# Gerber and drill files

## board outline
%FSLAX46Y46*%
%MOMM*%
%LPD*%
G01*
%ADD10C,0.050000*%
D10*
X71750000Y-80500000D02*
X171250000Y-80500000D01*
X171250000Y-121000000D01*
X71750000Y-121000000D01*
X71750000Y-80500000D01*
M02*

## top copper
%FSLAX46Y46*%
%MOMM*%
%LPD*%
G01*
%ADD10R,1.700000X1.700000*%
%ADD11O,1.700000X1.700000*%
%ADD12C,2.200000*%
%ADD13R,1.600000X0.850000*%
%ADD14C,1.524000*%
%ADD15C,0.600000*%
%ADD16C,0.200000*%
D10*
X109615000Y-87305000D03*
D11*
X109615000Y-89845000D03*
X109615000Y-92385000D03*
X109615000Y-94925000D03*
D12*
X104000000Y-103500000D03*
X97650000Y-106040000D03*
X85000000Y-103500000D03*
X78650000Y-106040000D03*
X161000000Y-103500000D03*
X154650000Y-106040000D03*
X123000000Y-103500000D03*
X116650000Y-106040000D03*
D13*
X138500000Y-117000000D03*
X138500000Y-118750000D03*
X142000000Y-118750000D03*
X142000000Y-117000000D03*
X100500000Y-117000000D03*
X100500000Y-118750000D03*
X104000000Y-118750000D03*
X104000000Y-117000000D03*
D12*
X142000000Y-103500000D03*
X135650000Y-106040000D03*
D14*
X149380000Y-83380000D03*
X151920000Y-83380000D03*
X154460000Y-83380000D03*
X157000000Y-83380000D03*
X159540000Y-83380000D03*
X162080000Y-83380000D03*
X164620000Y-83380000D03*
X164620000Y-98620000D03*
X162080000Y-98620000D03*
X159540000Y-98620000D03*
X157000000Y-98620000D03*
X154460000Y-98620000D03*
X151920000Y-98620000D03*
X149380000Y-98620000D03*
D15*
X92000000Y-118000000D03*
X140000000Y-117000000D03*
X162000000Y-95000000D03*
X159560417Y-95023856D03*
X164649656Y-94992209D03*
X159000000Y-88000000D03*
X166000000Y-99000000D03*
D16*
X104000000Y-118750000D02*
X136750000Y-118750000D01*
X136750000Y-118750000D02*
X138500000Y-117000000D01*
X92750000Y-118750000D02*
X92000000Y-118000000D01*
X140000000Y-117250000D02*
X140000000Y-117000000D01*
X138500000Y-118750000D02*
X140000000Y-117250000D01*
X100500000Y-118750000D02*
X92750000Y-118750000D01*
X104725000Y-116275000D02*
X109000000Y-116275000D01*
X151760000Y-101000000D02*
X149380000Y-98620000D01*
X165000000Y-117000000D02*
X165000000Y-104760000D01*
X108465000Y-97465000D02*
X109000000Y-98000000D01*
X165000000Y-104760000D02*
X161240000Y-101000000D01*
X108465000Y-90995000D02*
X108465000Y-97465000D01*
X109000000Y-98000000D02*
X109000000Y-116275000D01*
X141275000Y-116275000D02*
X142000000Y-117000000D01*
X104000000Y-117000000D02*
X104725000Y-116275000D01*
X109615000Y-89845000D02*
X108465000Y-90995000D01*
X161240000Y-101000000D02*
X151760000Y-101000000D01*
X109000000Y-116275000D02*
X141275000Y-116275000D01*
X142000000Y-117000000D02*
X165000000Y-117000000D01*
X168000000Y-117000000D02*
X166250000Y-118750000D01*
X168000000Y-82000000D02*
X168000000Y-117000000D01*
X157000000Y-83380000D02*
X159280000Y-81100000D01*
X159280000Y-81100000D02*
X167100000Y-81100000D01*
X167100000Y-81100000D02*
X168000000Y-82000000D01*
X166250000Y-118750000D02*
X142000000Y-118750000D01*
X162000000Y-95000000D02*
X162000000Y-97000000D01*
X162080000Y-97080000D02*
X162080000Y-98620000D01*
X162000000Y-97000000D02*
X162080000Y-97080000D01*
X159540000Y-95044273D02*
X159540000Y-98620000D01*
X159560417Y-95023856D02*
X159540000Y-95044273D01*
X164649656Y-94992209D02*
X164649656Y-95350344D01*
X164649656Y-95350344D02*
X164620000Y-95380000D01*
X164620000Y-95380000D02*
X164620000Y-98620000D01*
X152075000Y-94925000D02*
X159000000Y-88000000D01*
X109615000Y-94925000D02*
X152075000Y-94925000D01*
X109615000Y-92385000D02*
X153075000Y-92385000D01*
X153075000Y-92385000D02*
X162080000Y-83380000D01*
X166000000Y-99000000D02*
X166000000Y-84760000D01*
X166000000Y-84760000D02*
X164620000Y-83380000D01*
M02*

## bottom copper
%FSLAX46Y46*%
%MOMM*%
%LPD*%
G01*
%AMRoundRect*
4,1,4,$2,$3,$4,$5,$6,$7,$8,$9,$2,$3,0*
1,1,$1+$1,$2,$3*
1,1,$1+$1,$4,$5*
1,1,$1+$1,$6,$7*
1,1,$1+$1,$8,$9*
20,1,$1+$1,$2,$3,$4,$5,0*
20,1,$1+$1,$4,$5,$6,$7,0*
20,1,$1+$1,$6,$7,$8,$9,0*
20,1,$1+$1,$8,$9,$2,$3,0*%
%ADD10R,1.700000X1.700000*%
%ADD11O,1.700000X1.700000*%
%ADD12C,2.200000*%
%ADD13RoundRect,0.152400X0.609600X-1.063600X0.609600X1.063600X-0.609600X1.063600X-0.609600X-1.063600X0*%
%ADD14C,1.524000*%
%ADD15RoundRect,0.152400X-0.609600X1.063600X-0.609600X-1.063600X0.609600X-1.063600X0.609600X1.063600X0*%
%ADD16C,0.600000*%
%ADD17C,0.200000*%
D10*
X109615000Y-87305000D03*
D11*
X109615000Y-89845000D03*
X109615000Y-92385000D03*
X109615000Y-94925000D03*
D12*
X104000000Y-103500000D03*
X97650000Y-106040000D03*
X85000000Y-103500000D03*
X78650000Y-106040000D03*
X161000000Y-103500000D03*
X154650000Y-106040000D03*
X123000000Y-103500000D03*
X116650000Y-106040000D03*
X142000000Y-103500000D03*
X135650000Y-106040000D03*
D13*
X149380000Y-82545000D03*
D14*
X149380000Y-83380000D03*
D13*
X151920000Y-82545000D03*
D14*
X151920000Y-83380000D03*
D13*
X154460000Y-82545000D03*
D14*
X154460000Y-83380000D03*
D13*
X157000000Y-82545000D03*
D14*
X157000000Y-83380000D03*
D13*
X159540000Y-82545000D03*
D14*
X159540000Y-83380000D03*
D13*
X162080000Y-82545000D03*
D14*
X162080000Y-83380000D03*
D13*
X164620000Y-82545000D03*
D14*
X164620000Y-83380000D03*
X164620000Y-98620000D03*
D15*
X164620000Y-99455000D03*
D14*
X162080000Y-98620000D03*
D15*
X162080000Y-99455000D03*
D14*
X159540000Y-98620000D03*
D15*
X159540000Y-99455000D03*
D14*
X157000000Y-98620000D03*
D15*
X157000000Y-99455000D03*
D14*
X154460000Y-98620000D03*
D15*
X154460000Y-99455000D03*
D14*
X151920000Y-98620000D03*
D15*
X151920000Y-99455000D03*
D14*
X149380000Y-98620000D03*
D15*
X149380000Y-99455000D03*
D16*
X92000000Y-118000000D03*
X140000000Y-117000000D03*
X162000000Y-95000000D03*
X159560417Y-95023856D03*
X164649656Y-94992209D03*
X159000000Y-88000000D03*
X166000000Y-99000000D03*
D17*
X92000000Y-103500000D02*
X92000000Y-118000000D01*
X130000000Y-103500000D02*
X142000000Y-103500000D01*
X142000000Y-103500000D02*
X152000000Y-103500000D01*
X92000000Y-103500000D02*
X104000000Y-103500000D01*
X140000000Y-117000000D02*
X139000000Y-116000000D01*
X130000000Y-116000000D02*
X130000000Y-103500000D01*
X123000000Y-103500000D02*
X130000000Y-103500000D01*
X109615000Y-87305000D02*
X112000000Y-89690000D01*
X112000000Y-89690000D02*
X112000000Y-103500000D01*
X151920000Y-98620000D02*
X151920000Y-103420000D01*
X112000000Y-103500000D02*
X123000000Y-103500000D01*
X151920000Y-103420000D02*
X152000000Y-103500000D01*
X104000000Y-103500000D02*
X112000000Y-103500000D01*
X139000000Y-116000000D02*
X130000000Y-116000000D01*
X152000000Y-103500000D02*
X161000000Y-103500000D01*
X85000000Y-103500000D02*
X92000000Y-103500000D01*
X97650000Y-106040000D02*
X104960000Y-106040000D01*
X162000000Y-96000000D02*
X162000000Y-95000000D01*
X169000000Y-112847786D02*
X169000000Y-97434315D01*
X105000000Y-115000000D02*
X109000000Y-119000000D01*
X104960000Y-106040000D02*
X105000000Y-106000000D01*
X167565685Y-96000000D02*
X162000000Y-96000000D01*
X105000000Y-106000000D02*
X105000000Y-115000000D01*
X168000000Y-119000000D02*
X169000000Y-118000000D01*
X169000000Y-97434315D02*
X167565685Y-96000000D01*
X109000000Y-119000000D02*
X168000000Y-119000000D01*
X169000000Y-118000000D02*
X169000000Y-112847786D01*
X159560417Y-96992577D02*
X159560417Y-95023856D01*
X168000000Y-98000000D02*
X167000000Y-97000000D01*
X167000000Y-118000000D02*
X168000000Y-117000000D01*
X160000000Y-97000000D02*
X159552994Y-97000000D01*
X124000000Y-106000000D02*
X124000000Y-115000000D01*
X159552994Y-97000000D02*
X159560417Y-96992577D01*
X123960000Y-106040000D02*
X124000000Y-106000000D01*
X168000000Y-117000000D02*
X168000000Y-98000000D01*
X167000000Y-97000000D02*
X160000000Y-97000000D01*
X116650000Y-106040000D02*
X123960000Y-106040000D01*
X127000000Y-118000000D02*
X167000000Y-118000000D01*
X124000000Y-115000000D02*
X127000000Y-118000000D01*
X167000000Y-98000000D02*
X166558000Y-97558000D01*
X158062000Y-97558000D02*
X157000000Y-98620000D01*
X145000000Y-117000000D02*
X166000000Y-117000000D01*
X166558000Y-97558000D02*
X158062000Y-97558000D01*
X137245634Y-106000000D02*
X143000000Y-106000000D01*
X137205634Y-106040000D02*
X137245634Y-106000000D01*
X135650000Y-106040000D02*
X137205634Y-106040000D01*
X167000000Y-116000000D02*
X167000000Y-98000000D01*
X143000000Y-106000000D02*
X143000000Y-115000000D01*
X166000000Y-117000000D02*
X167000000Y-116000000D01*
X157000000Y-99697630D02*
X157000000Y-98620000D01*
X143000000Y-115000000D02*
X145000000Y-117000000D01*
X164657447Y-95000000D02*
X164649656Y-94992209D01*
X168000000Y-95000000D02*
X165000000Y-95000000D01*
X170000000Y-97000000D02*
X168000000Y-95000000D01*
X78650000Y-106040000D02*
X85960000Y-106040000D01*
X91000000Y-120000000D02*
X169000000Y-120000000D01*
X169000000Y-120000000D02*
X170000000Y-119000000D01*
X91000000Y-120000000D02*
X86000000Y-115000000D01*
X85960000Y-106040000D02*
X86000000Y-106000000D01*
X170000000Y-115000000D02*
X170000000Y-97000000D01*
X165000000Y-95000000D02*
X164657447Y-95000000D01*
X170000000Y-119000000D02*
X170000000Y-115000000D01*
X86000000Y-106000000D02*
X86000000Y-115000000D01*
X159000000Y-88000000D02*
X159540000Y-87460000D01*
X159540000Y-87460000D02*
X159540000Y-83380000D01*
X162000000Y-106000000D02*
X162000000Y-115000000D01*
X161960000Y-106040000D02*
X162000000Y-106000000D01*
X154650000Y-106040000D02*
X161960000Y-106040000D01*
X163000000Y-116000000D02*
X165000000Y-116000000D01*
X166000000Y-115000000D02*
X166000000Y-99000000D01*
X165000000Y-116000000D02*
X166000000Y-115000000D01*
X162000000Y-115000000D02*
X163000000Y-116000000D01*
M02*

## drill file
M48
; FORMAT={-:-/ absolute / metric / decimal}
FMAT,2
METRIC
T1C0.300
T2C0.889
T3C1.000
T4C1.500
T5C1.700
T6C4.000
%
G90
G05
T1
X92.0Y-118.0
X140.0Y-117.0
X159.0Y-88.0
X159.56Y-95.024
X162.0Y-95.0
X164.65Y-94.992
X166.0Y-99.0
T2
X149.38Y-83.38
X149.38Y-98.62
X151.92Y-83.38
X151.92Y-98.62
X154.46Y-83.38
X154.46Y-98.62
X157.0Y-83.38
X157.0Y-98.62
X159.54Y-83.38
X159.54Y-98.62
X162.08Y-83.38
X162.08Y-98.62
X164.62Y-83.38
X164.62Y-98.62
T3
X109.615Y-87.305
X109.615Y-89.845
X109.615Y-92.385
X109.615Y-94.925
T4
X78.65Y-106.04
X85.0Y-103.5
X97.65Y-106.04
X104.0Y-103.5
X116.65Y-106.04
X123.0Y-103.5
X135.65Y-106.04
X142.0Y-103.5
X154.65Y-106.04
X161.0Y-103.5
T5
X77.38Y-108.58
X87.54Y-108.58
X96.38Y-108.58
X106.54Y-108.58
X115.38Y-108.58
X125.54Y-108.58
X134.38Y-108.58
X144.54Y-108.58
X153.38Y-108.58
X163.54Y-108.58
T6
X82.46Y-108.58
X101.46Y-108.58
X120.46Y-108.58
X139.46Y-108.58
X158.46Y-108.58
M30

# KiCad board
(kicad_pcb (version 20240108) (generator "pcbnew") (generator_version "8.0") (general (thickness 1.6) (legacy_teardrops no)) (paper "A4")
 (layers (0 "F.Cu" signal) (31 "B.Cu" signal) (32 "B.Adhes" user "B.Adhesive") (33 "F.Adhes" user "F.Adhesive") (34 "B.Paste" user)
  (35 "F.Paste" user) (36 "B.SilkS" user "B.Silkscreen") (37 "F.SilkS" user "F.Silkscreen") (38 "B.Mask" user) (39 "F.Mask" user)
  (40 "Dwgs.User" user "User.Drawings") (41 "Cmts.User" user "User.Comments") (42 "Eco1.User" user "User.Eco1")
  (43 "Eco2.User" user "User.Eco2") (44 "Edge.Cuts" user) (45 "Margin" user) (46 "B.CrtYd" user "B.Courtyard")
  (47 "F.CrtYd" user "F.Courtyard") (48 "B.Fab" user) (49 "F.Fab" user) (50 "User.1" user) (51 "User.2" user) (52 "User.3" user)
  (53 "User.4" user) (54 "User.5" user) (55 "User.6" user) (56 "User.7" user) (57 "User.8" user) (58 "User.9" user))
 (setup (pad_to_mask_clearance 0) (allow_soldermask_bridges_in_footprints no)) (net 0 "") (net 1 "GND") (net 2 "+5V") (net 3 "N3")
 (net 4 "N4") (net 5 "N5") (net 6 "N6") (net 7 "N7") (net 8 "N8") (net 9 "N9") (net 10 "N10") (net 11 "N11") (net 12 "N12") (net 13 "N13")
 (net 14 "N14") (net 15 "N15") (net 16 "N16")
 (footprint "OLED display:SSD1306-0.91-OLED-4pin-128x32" (layer "F.Cu") (at 73.115 85.115)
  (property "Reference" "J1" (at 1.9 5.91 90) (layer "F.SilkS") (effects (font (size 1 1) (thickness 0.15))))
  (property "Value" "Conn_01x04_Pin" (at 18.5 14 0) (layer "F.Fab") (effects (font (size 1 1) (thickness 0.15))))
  (pad "1" thru_hole rect (at 36.5 2.19) (size 1.7 1.7) (drill 1) (layers "*.Cu" "*.Mask") (remove_unused_layers no) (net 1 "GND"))
  (pad "2" thru_hole oval (at 36.5 4.73) (size 1.7 1.7) (drill 1) (layers "*.Cu" "*.Mask") (remove_unused_layers no) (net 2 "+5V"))
  (pad "3" thru_hole oval (at 36.5 7.27) (size 1.7 1.7) (drill 1) (layers "*.Cu" "*.Mask") (remove_unused_layers no) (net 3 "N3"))
  (pad "4" thru_hole oval (at 36.5 9.81) (size 1.7 1.7) (drill 1) (layers "*.Cu" "*.Mask") (remove_unused_layers no) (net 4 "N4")))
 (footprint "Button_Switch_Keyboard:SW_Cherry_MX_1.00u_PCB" (layer "F.Cu") (at 104 103.5)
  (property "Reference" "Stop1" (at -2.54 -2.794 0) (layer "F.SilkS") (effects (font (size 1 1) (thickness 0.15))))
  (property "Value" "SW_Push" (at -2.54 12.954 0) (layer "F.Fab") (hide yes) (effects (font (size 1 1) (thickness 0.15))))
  (pad "" np_thru_hole circle (at -7.62 5.08) (size 1.7 1.7) (drill 1.7) (layers "*.Cu" "*.Mask"))
  (pad "" np_thru_hole circle (at -2.54 5.08) (size 4 4) (drill 4) (layers "*.Cu" "*.Mask"))
  (pad "" np_thru_hole circle (at 2.54 5.08) (size 1.7 1.7) (drill 1.7) (layers "*.Cu" "*.Mask"))
  (pad "1" thru_hole circle (at 0 0) (size 2.2 2.2) (drill 1.5) (layers "*.Cu" "*.Mask") (remove_unused_layers no) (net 1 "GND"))
  (pad "2" thru_hole circle (at -6.35 2.54) (size 2.2 2.2) (drill 1.5) (layers "*.Cu" "*.Mask") (remove_unused_layers no) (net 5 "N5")))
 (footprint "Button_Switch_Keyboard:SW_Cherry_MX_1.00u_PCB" (layer "F.Cu") (at 85 103.5)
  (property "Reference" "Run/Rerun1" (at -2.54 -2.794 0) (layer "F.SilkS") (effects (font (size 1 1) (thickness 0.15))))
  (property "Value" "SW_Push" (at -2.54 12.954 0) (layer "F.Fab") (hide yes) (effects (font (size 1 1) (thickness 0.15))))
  (pad "" np_thru_hole circle (at -7.62 5.08) (size 1.7 1.7) (drill 1.7) (layers "*.Cu" "*.Mask"))
  (pad "" np_thru_hole circle (at -2.54 5.08) (size 4 4) (drill 4) (layers "*.Cu" "*.Mask"))
  (pad "" np_thru_hole circle (at 2.54 5.08) (size 1.7 1.7) (drill 1.7) (layers "*.Cu" "*.Mask"))
  (pad "1" thru_hole circle (at 0 0) (size 2.2 2.2) (drill 1.5) (layers "*.Cu" "*.Mask") (remove_unused_layers no) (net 1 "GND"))
  (pad "2" thru_hole circle (at -6.35 2.54) (size 2.2 2.2) (drill 1.5) (layers "*.Cu" "*.Mask") (remove_unused_layers no) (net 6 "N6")))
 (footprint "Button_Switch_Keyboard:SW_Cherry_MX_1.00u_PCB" (layer "F.Cu") (at 161 103.5)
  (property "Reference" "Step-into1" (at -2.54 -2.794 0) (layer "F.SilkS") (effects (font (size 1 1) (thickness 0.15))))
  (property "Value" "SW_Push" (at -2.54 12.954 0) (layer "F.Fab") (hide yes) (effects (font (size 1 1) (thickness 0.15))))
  (pad "" np_thru_hole circle (at -7.62 5.08) (size 1.7 1.7) (drill 1.7) (layers "*.Cu" "*.Mask"))
  (pad "" np_thru_hole circle (at -2.54 5.08) (size 4 4) (drill 4) (layers "*.Cu" "*.Mask"))
  (pad "" np_thru_hole circle (at 2.54 5.08) (size 1.7 1.7) (drill 1.7) (layers "*.Cu" "*.Mask"))
  (pad "1" thru_hole circle (at 0 0) (size 2.2 2.2) (drill 1.5) (layers "*.Cu" "*.Mask") (remove_unused_layers no) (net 1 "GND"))
  (pad "2" thru_hole circle (at -6.35 2.54) (size 2.2 2.2) (drill 1.5) (layers "*.Cu" "*.Mask") (remove_unused_layers no) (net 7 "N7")))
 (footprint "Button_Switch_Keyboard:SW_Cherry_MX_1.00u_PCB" (layer "F.Cu") (at 123 103.5)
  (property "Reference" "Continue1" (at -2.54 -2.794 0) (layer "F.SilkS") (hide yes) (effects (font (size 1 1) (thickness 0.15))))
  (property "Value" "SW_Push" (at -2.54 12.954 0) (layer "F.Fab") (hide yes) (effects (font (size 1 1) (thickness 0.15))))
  (pad "" np_thru_hole circle (at -7.62 5.08) (size 1.7 1.7) (drill 1.7) (layers "*.Cu" "*.Mask"))
  (pad "" np_thru_hole circle (at -2.54 5.08) (size 4 4) (drill 4) (layers "*.Cu" "*.Mask"))
  (pad "" np_thru_hole circle (at 2.54 5.08) (size 1.7 1.7) (drill 1.7) (layers "*.Cu" "*.Mask"))
  (pad "1" thru_hole circle (at 0 0) (size 2.2 2.2) (drill 1.5) (layers "*.Cu" "*.Mask") (remove_unused_layers no) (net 1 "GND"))
  (pad "2" thru_hole circle (at -6.35 2.54) (size 2.2 2.2) (drill 1.5) (layers "*.Cu" "*.Mask") (remove_unused_layers no) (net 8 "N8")))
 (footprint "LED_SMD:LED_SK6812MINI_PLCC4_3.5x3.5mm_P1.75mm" (layer "F.Cu") (at 140.25 117.875)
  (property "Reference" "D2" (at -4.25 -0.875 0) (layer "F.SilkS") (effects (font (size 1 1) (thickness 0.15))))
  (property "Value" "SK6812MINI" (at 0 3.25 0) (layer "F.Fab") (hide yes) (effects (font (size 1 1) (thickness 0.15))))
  (pad "1" smd rect (at -1.75 -0.875) (size 1.6 0.85) (layers "F.Cu" "F.Paste" "F.Mask") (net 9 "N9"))
  (pad "2" smd rect (at -1.75 0.875) (size 1.6 0.85) (layers "F.Cu" "F.Paste" "F.Mask") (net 1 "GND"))
  (pad "3" smd rect (at 1.75 0.875) (size 1.6 0.85) (layers "F.Cu" "F.Paste" "F.Mask") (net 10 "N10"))
  (pad "4" smd rect (at 1.75 -0.875) (size 1.6 0.85) (layers "F.Cu" "F.Paste" "F.Mask") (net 2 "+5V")))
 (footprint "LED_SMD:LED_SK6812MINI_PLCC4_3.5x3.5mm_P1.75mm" (layer "F.Cu") (at 102.25 117.875)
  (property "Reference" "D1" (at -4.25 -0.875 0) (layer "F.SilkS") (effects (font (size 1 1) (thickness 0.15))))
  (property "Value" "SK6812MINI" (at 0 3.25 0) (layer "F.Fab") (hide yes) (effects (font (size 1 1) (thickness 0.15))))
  (pad "1" smd rect (at -1.75 -0.875) (size 1.6 0.85) (layers "F.Cu" "F.Paste" "F.Mask") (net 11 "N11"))
  (pad "2" smd rect (at -1.75 0.875) (size 1.6 0.85) (layers "F.Cu" "F.Paste" "F.Mask") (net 1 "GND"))
  (pad "3" smd rect (at 1.75 0.875) (size 1.6 0.85) (layers "F.Cu" "F.Paste" "F.Mask") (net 9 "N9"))
  (pad "4" smd rect (at 1.75 -0.875) (size 1.6 0.85) (layers "F.Cu" "F.Paste" "F.Mask") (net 2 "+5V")))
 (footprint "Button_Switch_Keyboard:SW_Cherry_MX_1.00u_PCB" (layer "F.Cu") (at 142 103.5)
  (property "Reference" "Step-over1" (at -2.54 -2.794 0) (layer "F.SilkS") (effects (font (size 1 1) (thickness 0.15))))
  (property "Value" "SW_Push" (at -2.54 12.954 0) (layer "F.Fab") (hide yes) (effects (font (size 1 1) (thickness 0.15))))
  (pad "" np_thru_hole circle (at -7.62 5.08) (size 1.7 1.7) (drill 1.7) (layers "*.Cu" "*.Mask"))
  (pad "" np_thru_hole circle (at -2.54 5.08) (size 4 4) (drill 4) (layers "*.Cu" "*.Mask"))
  (pad "" np_thru_hole circle (at 2.54 5.08) (size 1.7 1.7) (drill 1.7) (layers "*.Cu" "*.Mask"))
  (pad "1" thru_hole circle (at 0 0) (size 2.2 2.2) (drill 1.5) (layers "*.Cu" "*.Mask") (remove_unused_layers no) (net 1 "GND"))
  (pad "2" thru_hole circle (at -6.35 2.54) (size 2.2 2.2) (drill 1.5) (layers "*.Cu" "*.Mask") (remove_unused_layers no) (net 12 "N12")))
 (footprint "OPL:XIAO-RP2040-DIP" (layer "B.Cu") (at 157 91 -90)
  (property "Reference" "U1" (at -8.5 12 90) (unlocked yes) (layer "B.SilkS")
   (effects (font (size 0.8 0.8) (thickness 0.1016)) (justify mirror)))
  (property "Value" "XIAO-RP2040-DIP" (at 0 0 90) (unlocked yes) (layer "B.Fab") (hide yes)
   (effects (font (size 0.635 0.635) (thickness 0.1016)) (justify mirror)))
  (pad "1" smd roundrect (at -8.455 7.62 90) (size 2.432 1.524) (layers "B.Cu" "B.Mask") (roundrect_rratio 0.1) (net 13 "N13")
   (thermal_bridge_angle 45))
  (pad "1" thru_hole circle (at -7.62 7.62 90) (size 1.524 1.524) (drill 0.889) (layers "*.Cu" "*.Mask") (remove_unused_layers no)
   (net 13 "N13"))
  (pad "2" smd roundrect (at -8.455 5.08 90) (size 2.432 1.524) (layers "B.Cu" "B.Mask") (roundrect_rratio 0.1) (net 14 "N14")
   (thermal_bridge_angle 45))
  (pad "2" thru_hole circle (at -7.62 5.08 90) (size 1.524 1.524) (drill 0.889) (layers "*.Cu" "*.Mask") (remove_unused_layers no)
   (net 14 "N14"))
  (pad "3" smd roundrect (at -8.455 2.54 90) (size 2.432 1.524) (layers "B.Cu" "B.Mask") (roundrect_rratio 0.1) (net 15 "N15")
   (thermal_bridge_angle 45))
  (pad "3" thru_hole circle (at -7.62 2.54 90) (size 1.524 1.524) (drill 0.889) (layers "*.Cu" "*.Mask") (remove_unused_layers no)
   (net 15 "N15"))
  (pad "4" smd roundrect (at -8.455 0 90) (size 2.432 1.524) (layers "B.Cu" "B.Mask") (roundrect_rratio 0.1) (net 10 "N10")
   (thermal_bridge_angle 45))
  (pad "4" thru_hole circle (at -7.62 0 90) (size 1.524 1.524) (drill 0.889) (layers "*.Cu" "*.Mask") (remove_unused_layers no)
   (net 10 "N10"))
  (pad "5" smd roundrect (at -8.455 -2.54 90) (size 2.432 1.524) (layers "B.Cu" "B.Mask") (roundrect_rratio 0.1) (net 4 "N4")
   (thermal_bridge_angle 45))
  (pad "5" thru_hole circle (at -7.62 -2.54 90) (size 1.524 1.524) (drill 0.889) (layers "*.Cu" "*.Mask") (remove_unused_layers no)
   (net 4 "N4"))
  (pad "6" smd roundrect (at -8.455 -5.08 90) (size 2.432 1.524) (layers "B.Cu" "B.Mask") (roundrect_rratio 0.1) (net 3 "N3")
   (thermal_bridge_angle 45))
  (pad "6" thru_hole circle (at -7.62 -5.08 90) (size 1.524 1.524) (drill 0.889) (layers "*.Cu" "*.Mask") (remove_unused_layers no)
   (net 3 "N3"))
  (pad "7" smd roundrect (at -8.455 -7.62 90) (size 2.432 1.524) (layers "B.Cu" "B.Mask") (roundrect_rratio 0.1) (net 7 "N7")
   (thermal_bridge_angle 45))
  (pad "7" thru_hole circle (at -7.62 -7.62 90) (size 1.524 1.524) (drill 0.889) (layers "*.Cu" "*.Mask") (remove_unused_layers no)
   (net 7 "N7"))
  (pad "8" thru_hole circle (at 7.62 -7.62 270) (size 1.524 1.524) (drill 0.889) (layers "*.Cu" "*.Mask") (remove_unused_layers no)
   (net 6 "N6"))
  (pad "8" smd roundrect (at 8.455 -7.62 270) (size 2.432 1.524) (layers "B.Cu" "B.Mask") (roundrect_rratio 0.1) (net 6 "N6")
   (thermal_bridge_angle 45))
  (pad "9" thru_hole circle (at 7.62 -5.08 270) (size 1.524 1.524) (drill 0.889) (layers "*.Cu" "*.Mask") (remove_unused_layers no)
   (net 5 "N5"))
  (pad "9" smd roundrect (at 8.455 -5.08 270) (size 2.432 1.524) (layers "B.Cu" "B.Mask") (roundrect_rratio 0.1) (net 5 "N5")
   (thermal_bridge_angle 45))
  (pad "10" thru_hole circle (at 7.62 -2.54 270) (size 1.524 1.524) (drill 0.889) (layers "*.Cu" "*.Mask") (remove_unused_layers no)
   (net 8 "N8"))
  (pad "10" smd roundrect (at 8.455 -2.54 270) (size 2.432 1.524) (layers "B.Cu" "B.Mask") (roundrect_rratio 0.1) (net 8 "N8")
   (thermal_bridge_angle 45))
  (pad "11" thru_hole circle (at 7.62 0 270) (size 1.524 1.524) (drill 0.889) (layers "*.Cu" "*.Mask") (remove_unused_layers no)
   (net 12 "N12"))
  (pad "11" smd roundrect (at 8.455 0 270) (size 2.432 1.524) (layers "B.Cu" "B.Mask") (roundrect_rratio 0.1) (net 12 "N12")
   (thermal_bridge_angle 45))
  (pad "12" thru_hole circle (at 7.62 2.54 270) (size 1.524 1.524) (drill 0.889) (layers "*.Cu" "*.Mask") (remove_unused_layers no)
   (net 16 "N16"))
  (pad "12" smd roundrect (at 8.455 2.54 270) (size 2.432 1.524) (layers "B.Cu" "B.Mask") (roundrect_rratio 0.1) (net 16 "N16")
   (thermal_bridge_angle 45))
  (pad "13" thru_hole circle (at 7.62 5.08 270) (size 1.524 1.524) (drill 0.889) (layers "*.Cu" "*.Mask") (remove_unused_layers no)
   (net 1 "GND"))
  (pad "13" smd roundrect (at 8.455 5.08 270) (size 2.432 1.524) (layers "B.Cu" "B.Mask") (roundrect_rratio 0.1) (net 1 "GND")
   (thermal_bridge_angle 45))
  (pad "14" thru_hole circle (at 7.62 7.62 270) (size 1.524 1.524) (drill 0.889) (layers "*.Cu" "*.Mask") (remove_unused_layers no)
   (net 2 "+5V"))
  (pad "14" smd roundrect (at 8.455 7.62 270) (size 2.432 1.524) (layers "B.Cu" "B.Mask") (roundrect_rratio 0.1) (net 2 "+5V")
   (thermal_bridge_angle 45)))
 (gr_rect (start 71.75 80.5) (end 171.25 121) (stroke (width 0.05) (type default)) (fill none) (layer "Edge.Cuts"))
 (segment (start 104 118.75) (end 136.75 118.75) (width 0.2) (layer "F.Cu") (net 9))
 (segment (start 136.75 118.75) (end 138.5 117) (width 0.2) (layer "F.Cu") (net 9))
 (segment (start 92.75 118.75) (end 92 118) (width 0.2) (layer "F.Cu") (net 1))
 (segment (start 140 117.25) (end 140 117) (width 0.2) (layer "F.Cu") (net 1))
 (segment (start 138.5 118.75) (end 140 117.25) (width 0.2) (layer "F.Cu") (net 1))
 (segment (start 100.5 118.75) (end 92.75 118.75) (width 0.2) (layer "F.Cu") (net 1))
 (via (at 92 118) (size 0.6) (drill 0.3) (layers "F.Cu" "B.Cu") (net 1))
 (via (at 140 117) (size 0.6) (drill 0.3) (layers "F.Cu" "B.Cu") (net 1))
 (segment (start 92 103.5) (end 92 118) (width 0.2) (layer "B.Cu") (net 1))
 (segment (start 130 103.5) (end 142 103.5) (width 0.2) (layer "B.Cu") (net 1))
 (segment (start 142 103.5) (end 152 103.5) (width 0.2) (layer "B.Cu") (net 1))
 (segment (start 92 103.5) (end 104 103.5) (width 0.2) (layer "B.Cu") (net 1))
 (segment (start 140 117) (end 139 116) (width 0.2) (layer "B.Cu") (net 1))
 (segment (start 130 116) (end 130 103.5) (width 0.2) (layer "B.Cu") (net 1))
 (segment (start 123 103.5) (end 130 103.5) (width 0.2) (layer "B.Cu") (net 1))
 (segment (start 109.615 87.305) (end 112 89.69) (width 0.2) (layer "B.Cu") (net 1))
 (segment (start 112 89.69) (end 112 103.5) (width 0.2) (layer "B.Cu") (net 1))
 (segment (start 151.92 98.62) (end 151.92 103.42) (width 0.2) (layer "B.Cu") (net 1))
 (segment (start 112 103.5) (end 123 103.5) (width 0.2) (layer "B.Cu") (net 1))
 (segment (start 151.92 103.42) (end 152 103.5) (width 0.2) (layer "B.Cu") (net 1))
 (segment (start 104 103.5) (end 112 103.5) (width 0.2) (layer "B.Cu") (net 1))
 (segment (start 139 116) (end 130 116) (width 0.2) (layer "B.Cu") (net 1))
 (segment (start 152 103.5) (end 161 103.5) (width 0.2) (layer "B.Cu") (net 1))
 (segment (start 85 103.5) (end 92 103.5) (width 0.2) (layer "B.Cu") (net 1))
 (segment (start 104.725 116.275) (end 109 116.275) (width 0.2) (layer "F.Cu") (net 2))
 (segment (start 151.76 101) (end 149.38 98.62) (width 0.2) (layer "F.Cu") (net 2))
 (segment (start 165 117) (end 165 104.76) (width 0.2) (layer "F.Cu") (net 2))
 (segment (start 108.465 97.465) (end 109 98) (width 0.2) (layer "F.Cu") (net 2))
 (segment (start 165 104.76) (end 161.24 101) (width 0.2) (layer "F.Cu") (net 2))
 (segment (start 108.465 90.995) (end 108.465 97.465) (width 0.2) (layer "F.Cu") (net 2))
 (segment (start 109 98) (end 109 116.275) (width 0.2) (layer "F.Cu") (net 2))
 (segment (start 141.275 116.275) (end 142 117) (width 0.2) (layer "F.Cu") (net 2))
 (segment (start 104 117) (end 104.725 116.275) (width 0.2) (layer "F.Cu") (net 2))
 (segment (start 109.615 89.845) (end 108.465 90.995) (width 0.2) (layer "F.Cu") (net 2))
 (segment (start 161.24 101) (end 151.76 101) (width 0.2) (layer "F.Cu") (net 2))
 (segment (start 109 116.275) (end 141.275 116.275) (width 0.2) (layer "F.Cu") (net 2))
 (segment (start 142 117) (end 165 117) (width 0.2) (layer "F.Cu") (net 2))
 (segment (start 168 117) (end 166.25 118.75) (width 0.2) (layer "F.Cu") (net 10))
 (segment (start 168 82) (end 168 117) (width 0.2) (layer "F.Cu") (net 10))
 (segment (start 157 83.38) (end 159.28 81.1) (width 0.2) (layer "F.Cu") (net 10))
 (segment (start 159.28 81.1) (end 167.1 81.1) (width 0.2) (layer "F.Cu") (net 10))
 (segment (start 167.1 81.1) (end 168 82) (width 0.2) (layer "F.Cu") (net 10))
 (segment (start 166.25 118.75) (end 142 118.75) (width 0.2) (layer "F.Cu") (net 10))
 (segment (start 162 95) (end 162 97) (width 0.2) (layer "F.Cu") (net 5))
 (segment (start 162.08 97.08) (end 162.08 98.62) (width 0.2) (layer "F.Cu") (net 5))
 (segment (start 162 97) (end 162.08 97.08) (width 0.2) (layer "F.Cu") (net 5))
 (via (at 162 95) (size 0.6) (drill 0.3) (layers "F.Cu" "B.Cu") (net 5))
 (segment (start 97.65 106.04) (end 104.96 106.04) (width 0.2) (layer "B.Cu") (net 5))
 (segment (start 162 96) (end 162 95) (width 0.2) (layer "B.Cu") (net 5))
 (segment (start 169 112.847786) (end 169 97.434315) (width 0.2) (layer "B.Cu") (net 5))
 (segment (start 105 115) (end 109 119) (width 0.2) (layer "B.Cu") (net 5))
 (segment (start 104.96 106.04) (end 105 106) (width 0.2) (layer "B.Cu") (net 5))
 (segment (start 167.565685 96) (end 162 96) (width 0.2) (layer "B.Cu") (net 5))
 (segment (start 105 106) (end 105 115) (width 0.2) (layer "B.Cu") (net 5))
 (segment (start 168 119) (end 169 118) (width 0.2) (layer "B.Cu") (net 5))
 (segment (start 169 97.434315) (end 167.565685 96) (width 0.2) (layer "B.Cu") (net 5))
 (segment (start 109 119) (end 168 119) (width 0.2) (layer "B.Cu") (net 5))
 (segment (start 169 118) (end 169 112.847786) (width 0.2) (layer "B.Cu") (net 5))
 (segment (start 159.54 95.044273) (end 159.54 98.62) (width 0.2) (layer "F.Cu") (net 8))
 (segment (start 159.560417 95.023856) (end 159.54 95.044273) (width 0.2) (layer "F.Cu") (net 8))
 (via (at 159.560417 95.023856) (size 0.6) (drill 0.3) (layers "F.Cu" "B.Cu") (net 8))
 (segment (start 159.560417 96.992577) (end 159.560417 95.023856) (width 0.2) (layer "B.Cu") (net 8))
 (segment (start 168 98) (end 167 97) (width 0.2) (layer "B.Cu") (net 8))
 (segment (start 167 118) (end 168 117) (width 0.2) (layer "B.Cu") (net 8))
 (segment (start 160 97) (end 159.552994 97) (width 0.2) (layer "B.Cu") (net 8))
 (segment (start 124 106) (end 124 115) (width 0.2) (layer "B.Cu") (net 8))
 (segment (start 159.552994 97) (end 159.560417 96.992577) (width 0.2) (layer "B.Cu") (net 8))
 (segment (start 123.96 106.04) (end 124 106) (width 0.2) (layer "B.Cu") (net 8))
 (segment (start 168 117) (end 168 98) (width 0.2) (layer "B.Cu") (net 8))
 (segment (start 167 97) (end 160 97) (width 0.2) (layer "B.Cu") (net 8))
 (segment (start 116.65 106.04) (end 123.96 106.04) (width 0.2) (layer "B.Cu") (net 8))
 (segment (start 127 118) (end 167 118) (width 0.2) (layer "B.Cu") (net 8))
 (segment (start 124 115) (end 127 118) (width 0.2) (layer "B.Cu") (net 8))
 (segment (start 167 98) (end 166.558 97.558) (width 0.2) (layer "B.Cu") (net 12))
 (segment (start 158.062 97.558) (end 157 98.62) (width 0.2) (layer "B.Cu") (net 12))
 (segment (start 145 117) (end 166 117) (width 0.2) (layer "B.Cu") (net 12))
 (segment (start 166.558 97.558) (end 158.062 97.558) (width 0.2) (layer "B.Cu") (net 12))
 (segment (start 137.245634 106) (end 143 106) (width 0.2) (layer "B.Cu") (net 12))
 (segment (start 137.205634 106.04) (end 137.245634 106) (width 0.2) (layer "B.Cu") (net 12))
 (segment (start 135.65 106.04) (end 137.205634 106.04) (width 0.2) (layer "B.Cu") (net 12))
 (segment (start 167 116) (end 167 98) (width 0.2) (layer "B.Cu") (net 12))
 (segment (start 143 106) (end 143 115) (width 0.2) (layer "B.Cu") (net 12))
 (segment (start 166 117) (end 167 116) (width 0.2) (layer "B.Cu") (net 12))
 (segment (start 157 99.69763) (end 157 98.62) (width 0.2) (layer "B.Cu") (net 12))
 (segment (start 143 115) (end 145 117) (width 0.2) (layer "B.Cu") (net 12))
 (segment (start 164.649656 94.992209) (end 164.649656 95.350344) (width 0.2) (layer "F.Cu") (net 6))
 (segment (start 164.649656 95.350344) (end 164.62 95.38) (width 0.2) (layer "F.Cu") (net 6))
 (segment (start 164.62 95.38) (end 164.62 98.62) (width 0.2) (layer "F.Cu") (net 6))
 (via (at 164.649656 94.992209) (size 0.6) (drill 0.3) (layers "F.Cu" "B.Cu") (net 6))
 (segment (start 164.657447 95) (end 164.649656 94.992209) (width 0.2) (layer "B.Cu") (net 6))
 (segment (start 168 95) (end 165 95) (width 0.2) (layer "B.Cu") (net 6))
 (segment (start 170 97) (end 168 95) (width 0.2) (layer "B.Cu") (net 6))
 (segment (start 78.65 106.04) (end 85.96 106.04) (width 0.2) (layer "B.Cu") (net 6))
 (segment (start 91 120) (end 169 120) (width 0.2) (layer "B.Cu") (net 6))
 (segment (start 169 120) (end 170 119) (width 0.2) (layer "B.Cu") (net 6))
 (segment (start 91 120) (end 86 115) (width 0.2) (layer "B.Cu") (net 6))
 (segment (start 85.96 106.04) (end 86 106) (width 0.2) (layer "B.Cu") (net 6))
 (segment (start 170 115) (end 170 97) (width 0.2) (layer "B.Cu") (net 6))
 (segment (start 165 95) (end 164.657447 95) (width 0.2) (layer "B.Cu") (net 6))
 (segment (start 170 119) (end 170 115) (width 0.2) (layer "B.Cu") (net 6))
 (segment (start 86 106) (end 86 115) (width 0.2) (layer "B.Cu") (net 6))
 (segment (start 152.075 94.925) (end 159 88) (width 0.2) (layer "F.Cu") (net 4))
 (segment (start 109.615 94.925) (end 152.075 94.925) (width 0.2) (layer "F.Cu") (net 4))
 (via (at 159 88) (size 0.6) (drill 0.3) (layers "F.Cu" "B.Cu") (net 4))
 (segment (start 159 88) (end 159.54 87.46) (width 0.2) (layer "B.Cu") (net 4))
 (segment (start 159.54 87.46) (end 159.54 83.38) (width 0.2) (layer "B.Cu") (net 4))
 (segment (start 109.615 92.385) (end 153.075 92.385) (width 0.2) (layer "F.Cu") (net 3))
 (segment (start 153.075 92.385) (end 162.08 83.38) (width 0.2) (layer "F.Cu") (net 3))
 (segment (start 166 99) (end 166 84.76) (width 0.2) (layer "F.Cu") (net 7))
 (segment (start 166 84.76) (end 164.62 83.38) (width 0.2) (layer "F.Cu") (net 7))
 (via (at 166 99) (size 0.6) (drill 0.3) (layers "F.Cu" "B.Cu") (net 7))
 (segment (start 162 106) (end 162 115) (width 0.2) (layer "B.Cu") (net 7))
 (segment (start 161.96 106.04) (end 162 106) (width 0.2) (layer "B.Cu") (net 7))
 (segment (start 154.65 106.04) (end 161.96 106.04) (width 0.2) (layer "B.Cu") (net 7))
 (segment (start 163 116) (end 165 116) (width 0.2) (layer "B.Cu") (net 7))
 (segment (start 166 115) (end 166 99) (width 0.2) (layer "B.Cu") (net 7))
 (segment (start 165 116) (end 166 115) (width 0.2) (layer "B.Cu") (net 7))
 (segment (start 162 115) (end 163 116) (width 0.2) (layer "B.Cu") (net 7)))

